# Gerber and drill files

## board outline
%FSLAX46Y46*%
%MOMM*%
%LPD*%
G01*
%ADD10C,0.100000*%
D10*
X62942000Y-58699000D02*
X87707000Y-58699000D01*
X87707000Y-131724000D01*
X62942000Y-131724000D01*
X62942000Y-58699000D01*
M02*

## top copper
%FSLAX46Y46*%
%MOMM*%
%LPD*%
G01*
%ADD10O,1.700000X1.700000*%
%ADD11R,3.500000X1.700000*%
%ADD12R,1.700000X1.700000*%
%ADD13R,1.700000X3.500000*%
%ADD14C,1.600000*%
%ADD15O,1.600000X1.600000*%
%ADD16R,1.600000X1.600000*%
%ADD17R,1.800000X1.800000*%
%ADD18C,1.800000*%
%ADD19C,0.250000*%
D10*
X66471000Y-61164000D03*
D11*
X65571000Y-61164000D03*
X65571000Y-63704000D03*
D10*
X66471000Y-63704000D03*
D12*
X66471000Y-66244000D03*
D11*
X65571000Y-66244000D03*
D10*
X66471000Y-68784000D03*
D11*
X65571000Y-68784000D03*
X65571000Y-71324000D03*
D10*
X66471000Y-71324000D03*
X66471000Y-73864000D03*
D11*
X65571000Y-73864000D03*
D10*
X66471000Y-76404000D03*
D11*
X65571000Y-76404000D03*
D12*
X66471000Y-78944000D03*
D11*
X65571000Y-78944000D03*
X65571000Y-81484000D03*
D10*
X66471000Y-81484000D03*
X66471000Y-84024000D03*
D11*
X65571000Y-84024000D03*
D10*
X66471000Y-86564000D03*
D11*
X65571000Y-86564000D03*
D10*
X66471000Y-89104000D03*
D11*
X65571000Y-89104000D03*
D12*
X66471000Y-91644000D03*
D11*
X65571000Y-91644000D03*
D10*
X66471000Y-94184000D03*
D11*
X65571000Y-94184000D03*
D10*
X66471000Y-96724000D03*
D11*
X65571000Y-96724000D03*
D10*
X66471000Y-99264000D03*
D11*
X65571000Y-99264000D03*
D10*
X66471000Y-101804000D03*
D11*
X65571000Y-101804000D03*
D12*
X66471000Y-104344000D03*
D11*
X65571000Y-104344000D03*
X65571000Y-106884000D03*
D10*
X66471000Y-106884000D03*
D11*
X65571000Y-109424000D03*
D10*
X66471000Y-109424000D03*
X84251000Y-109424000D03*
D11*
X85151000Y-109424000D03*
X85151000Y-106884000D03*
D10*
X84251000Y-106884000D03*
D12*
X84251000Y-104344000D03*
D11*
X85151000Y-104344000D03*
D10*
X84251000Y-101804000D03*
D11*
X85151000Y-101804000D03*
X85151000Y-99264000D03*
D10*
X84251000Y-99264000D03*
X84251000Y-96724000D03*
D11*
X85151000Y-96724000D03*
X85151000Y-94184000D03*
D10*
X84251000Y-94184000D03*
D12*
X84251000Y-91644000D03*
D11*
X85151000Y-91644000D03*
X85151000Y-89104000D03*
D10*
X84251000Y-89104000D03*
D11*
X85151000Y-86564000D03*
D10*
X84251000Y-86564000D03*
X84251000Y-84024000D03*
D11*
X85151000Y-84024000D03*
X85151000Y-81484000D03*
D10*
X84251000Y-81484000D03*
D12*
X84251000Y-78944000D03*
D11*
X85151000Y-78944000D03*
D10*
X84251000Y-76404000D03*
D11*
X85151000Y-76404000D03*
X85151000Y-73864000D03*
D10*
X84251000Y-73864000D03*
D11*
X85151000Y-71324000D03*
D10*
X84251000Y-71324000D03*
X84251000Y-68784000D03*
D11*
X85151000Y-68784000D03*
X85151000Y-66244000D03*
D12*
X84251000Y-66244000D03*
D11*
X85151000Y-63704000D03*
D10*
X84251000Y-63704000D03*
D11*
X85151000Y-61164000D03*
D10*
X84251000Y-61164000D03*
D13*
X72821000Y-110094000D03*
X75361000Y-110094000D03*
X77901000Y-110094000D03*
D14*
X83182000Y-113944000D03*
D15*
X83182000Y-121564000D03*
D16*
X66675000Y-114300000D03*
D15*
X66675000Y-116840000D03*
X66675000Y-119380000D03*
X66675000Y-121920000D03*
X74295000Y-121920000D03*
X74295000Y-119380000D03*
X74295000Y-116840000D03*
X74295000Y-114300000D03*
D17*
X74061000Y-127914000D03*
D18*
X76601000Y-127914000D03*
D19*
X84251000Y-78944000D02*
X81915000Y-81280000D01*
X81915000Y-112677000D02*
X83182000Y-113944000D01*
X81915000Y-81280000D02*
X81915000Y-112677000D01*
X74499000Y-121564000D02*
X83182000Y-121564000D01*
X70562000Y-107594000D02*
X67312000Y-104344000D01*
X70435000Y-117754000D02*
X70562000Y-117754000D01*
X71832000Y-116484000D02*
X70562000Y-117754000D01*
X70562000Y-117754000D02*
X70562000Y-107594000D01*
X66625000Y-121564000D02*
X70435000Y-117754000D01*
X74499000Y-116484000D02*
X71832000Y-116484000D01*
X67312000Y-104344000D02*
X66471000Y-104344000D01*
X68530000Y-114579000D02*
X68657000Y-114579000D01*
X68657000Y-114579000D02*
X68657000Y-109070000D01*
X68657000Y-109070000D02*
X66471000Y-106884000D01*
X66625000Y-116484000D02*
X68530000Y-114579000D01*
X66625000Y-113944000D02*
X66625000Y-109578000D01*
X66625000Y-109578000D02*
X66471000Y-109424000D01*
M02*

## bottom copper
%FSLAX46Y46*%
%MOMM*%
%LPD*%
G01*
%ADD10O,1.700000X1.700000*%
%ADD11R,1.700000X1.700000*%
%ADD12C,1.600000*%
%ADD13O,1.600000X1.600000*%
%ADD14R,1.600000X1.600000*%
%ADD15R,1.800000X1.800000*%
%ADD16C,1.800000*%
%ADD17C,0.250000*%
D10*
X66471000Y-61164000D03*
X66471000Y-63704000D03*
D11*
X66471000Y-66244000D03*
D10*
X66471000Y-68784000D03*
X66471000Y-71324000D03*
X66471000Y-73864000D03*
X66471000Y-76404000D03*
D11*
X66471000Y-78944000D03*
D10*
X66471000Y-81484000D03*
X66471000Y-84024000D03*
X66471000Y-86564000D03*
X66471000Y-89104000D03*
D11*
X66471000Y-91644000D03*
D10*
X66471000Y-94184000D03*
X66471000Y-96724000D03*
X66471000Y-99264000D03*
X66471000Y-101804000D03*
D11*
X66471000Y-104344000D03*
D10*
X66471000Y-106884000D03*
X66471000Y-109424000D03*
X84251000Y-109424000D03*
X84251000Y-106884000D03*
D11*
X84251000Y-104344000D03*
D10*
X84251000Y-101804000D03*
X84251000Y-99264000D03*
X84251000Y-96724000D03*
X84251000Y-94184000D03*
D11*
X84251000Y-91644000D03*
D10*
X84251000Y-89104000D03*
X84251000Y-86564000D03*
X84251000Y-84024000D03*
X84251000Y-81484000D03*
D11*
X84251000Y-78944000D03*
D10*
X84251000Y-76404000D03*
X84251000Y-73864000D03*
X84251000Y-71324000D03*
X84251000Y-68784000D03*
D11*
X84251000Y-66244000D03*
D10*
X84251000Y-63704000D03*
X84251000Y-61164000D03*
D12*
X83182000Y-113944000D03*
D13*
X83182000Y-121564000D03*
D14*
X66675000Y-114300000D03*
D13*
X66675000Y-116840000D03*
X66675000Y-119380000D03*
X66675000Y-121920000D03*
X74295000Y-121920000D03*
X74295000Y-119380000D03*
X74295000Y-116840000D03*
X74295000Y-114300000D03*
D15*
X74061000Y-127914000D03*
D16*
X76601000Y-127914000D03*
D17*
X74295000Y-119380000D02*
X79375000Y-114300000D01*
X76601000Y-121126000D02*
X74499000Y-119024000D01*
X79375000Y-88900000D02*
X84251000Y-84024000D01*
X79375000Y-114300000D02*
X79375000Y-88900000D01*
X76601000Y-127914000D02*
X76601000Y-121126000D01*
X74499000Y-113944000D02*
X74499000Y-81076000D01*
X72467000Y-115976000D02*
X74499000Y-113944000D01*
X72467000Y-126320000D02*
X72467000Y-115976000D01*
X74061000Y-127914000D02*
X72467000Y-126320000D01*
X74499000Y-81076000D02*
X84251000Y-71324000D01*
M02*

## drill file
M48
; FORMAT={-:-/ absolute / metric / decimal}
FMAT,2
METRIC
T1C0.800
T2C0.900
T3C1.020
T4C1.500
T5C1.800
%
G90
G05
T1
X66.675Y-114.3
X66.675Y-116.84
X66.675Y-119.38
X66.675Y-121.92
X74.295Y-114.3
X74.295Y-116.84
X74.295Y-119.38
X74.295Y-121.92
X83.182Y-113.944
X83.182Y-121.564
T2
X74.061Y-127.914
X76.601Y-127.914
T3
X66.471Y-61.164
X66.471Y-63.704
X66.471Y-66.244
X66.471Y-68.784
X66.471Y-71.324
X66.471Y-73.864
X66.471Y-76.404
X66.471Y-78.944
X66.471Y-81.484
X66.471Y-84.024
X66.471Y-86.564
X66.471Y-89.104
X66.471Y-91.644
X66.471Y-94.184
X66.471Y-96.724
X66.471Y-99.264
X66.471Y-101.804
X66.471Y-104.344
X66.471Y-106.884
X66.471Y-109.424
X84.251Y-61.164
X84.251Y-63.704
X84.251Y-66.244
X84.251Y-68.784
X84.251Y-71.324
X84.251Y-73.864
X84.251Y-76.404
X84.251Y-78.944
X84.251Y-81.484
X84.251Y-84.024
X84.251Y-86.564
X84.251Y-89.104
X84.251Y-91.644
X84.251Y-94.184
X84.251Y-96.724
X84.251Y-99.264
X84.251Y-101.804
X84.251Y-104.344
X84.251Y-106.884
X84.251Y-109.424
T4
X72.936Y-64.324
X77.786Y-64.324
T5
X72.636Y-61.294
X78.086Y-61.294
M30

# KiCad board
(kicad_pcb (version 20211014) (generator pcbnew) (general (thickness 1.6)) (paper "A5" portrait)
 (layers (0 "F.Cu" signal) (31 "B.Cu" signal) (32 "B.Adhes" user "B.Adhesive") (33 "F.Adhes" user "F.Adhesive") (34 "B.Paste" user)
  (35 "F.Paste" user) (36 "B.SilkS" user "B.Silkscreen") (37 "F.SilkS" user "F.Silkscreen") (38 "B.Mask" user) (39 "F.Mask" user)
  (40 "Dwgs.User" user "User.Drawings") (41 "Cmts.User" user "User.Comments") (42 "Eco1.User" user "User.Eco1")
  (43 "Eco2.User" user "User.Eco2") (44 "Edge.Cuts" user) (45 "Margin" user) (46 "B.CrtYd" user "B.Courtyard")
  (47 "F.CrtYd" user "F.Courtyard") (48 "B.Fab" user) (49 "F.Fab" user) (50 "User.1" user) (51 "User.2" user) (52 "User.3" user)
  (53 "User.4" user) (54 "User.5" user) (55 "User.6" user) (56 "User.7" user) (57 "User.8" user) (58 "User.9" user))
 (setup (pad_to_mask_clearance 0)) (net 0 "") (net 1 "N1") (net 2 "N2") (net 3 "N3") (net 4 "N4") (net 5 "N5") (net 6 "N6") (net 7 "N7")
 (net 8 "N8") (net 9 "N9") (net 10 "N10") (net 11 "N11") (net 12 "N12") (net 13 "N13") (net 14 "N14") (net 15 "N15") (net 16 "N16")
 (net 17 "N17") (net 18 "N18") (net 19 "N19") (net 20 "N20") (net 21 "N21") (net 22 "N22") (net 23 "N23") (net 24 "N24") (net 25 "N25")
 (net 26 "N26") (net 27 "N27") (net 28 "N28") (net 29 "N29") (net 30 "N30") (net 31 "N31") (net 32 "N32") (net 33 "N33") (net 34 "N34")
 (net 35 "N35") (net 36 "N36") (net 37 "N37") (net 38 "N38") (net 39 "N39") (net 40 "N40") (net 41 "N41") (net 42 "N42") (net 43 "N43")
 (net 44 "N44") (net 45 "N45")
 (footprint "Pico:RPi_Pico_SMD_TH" (layer "F.Cu") (at 75.361 85.294)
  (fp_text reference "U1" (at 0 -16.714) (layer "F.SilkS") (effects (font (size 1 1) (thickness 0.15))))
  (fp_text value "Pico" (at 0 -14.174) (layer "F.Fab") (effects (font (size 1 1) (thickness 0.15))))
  (pad "" np_thru_hole oval (at -2.425 -20.97) (size 1.5 1.5) (drill 1.5) (layers *.Cu *.Mask))
  (pad "" np_thru_hole oval (at 2.725 -24) (size 1.8 1.8) (drill 1.8) (layers *.Cu *.Mask))
  (pad "" np_thru_hole oval (at 2.425 -20.97) (size 1.5 1.5) (drill 1.5) (layers *.Cu *.Mask))
  (pad "" np_thru_hole oval (at -2.725 -24) (size 1.8 1.8) (drill 1.8) (layers *.Cu *.Mask))
  (pad "1" thru_hole oval (at -8.89 -24.13) (size 1.7 1.7) (drill 1.02) (layers *.Cu *.Mask) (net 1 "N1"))
  (pad "1" smd rect (at -8.89 -24.13) (size 3.5 1.7) (drill (offset -0.9 0)) (layers "F.Cu" "F.Mask") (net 1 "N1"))
  (pad "2" smd rect (at -8.89 -21.59) (size 3.5 1.7) (drill (offset -0.9 0)) (layers "F.Cu" "F.Mask") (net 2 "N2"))
  (pad "2" thru_hole oval (at -8.89 -21.59) (size 1.7 1.7) (drill 1.02) (layers *.Cu *.Mask) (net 2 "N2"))
  (pad "3" thru_hole rect (at -8.89 -19.05) (size 1.7 1.7) (drill 1.02) (layers *.Cu *.Mask) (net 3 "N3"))
  (pad "3" smd rect (at -8.89 -19.05) (size 3.5 1.7) (drill (offset -0.9 0)) (layers "F.Cu" "F.Mask") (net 3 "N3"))
  (pad "4" thru_hole oval (at -8.89 -16.51) (size 1.7 1.7) (drill 1.02) (layers *.Cu *.Mask) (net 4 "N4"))
  (pad "4" smd rect (at -8.89 -16.51) (size 3.5 1.7) (drill (offset -0.9 0)) (layers "F.Cu" "F.Mask") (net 4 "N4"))
  (pad "5" smd rect (at -8.89 -13.97) (size 3.5 1.7) (drill (offset -0.9 0)) (layers "F.Cu" "F.Mask") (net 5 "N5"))
  (pad "5" thru_hole oval (at -8.89 -13.97) (size 1.7 1.7) (drill 1.02) (layers *.Cu *.Mask) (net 5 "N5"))
  (pad "6" thru_hole oval (at -8.89 -11.43) (size 1.7 1.7) (drill 1.02) (layers *.Cu *.Mask) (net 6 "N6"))
  (pad "6" smd rect (at -8.89 -11.43) (size 3.5 1.7) (drill (offset -0.9 0)) (layers "F.Cu" "F.Mask") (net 6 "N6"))
  (pad "7" thru_hole oval (at -8.89 -8.89) (size 1.7 1.7) (drill 1.02) (layers *.Cu *.Mask) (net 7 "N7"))
  (pad "7" smd rect (at -8.89 -8.89) (size 3.5 1.7) (drill (offset -0.9 0)) (layers "F.Cu" "F.Mask") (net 7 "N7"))
  (pad "8" thru_hole rect (at -8.89 -6.35) (size 1.7 1.7) (drill 1.02) (layers *.Cu *.Mask) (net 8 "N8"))
  (pad "8" smd rect (at -8.89 -6.35) (size 3.5 1.7) (drill (offset -0.9 0)) (layers "F.Cu" "F.Mask") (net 8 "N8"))
  (pad "9" smd rect (at -8.89 -3.81) (size 3.5 1.7) (drill (offset -0.9 0)) (layers "F.Cu" "F.Mask") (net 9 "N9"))
  (pad "9" thru_hole oval (at -8.89 -3.81) (size 1.7 1.7) (drill 1.02) (layers *.Cu *.Mask) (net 9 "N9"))
  (pad "10" thru_hole oval (at -8.89 -1.27) (size 1.7 1.7) (drill 1.02) (layers *.Cu *.Mask) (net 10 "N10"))
  (pad "10" smd rect (at -8.89 -1.27) (size 3.5 1.7) (drill (offset -0.9 0)) (layers "F.Cu" "F.Mask") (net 10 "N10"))
  (pad "11" thru_hole oval (at -8.89 1.27) (size 1.7 1.7) (drill 1.02) (layers *.Cu *.Mask) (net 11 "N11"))
  (pad "11" smd rect (at -8.89 1.27) (size 3.5 1.7) (drill (offset -0.9 0)) (layers "F.Cu" "F.Mask") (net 11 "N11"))
  (pad "12" thru_hole oval (at -8.89 3.81) (size 1.7 1.7) (drill 1.02) (layers *.Cu *.Mask) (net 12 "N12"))
  (pad "12" smd rect (at -8.89 3.81) (size 3.5 1.7) (drill (offset -0.9 0)) (layers "F.Cu" "F.Mask") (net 12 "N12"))
  (pad "13" thru_hole rect (at -8.89 6.35) (size 1.7 1.7) (drill 1.02) (layers *.Cu *.Mask) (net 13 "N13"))
  (pad "13" smd rect (at -8.89 6.35) (size 3.5 1.7) (drill (offset -0.9 0)) (layers "F.Cu" "F.Mask") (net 13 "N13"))
  (pad "14" thru_hole oval (at -8.89 8.89) (size 1.7 1.7) (drill 1.02) (layers *.Cu *.Mask) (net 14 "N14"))
  (pad "14" smd rect (at -8.89 8.89) (size 3.5 1.7) (drill (offset -0.9 0)) (layers "F.Cu" "F.Mask") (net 14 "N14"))
  (pad "15" thru_hole oval (at -8.89 11.43) (size 1.7 1.7) (drill 1.02) (layers *.Cu *.Mask) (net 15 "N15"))
  (pad "15" smd rect (at -8.89 11.43) (size 3.5 1.7) (drill (offset -0.9 0)) (layers "F.Cu" "F.Mask") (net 15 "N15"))
  (pad "16" thru_hole oval (at -8.89 13.97) (size 1.7 1.7) (drill 1.02) (layers *.Cu *.Mask) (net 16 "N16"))
  (pad "16" smd rect (at -8.89 13.97) (size 3.5 1.7) (drill (offset -0.9 0)) (layers "F.Cu" "F.Mask") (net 16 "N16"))
  (pad "17" thru_hole oval (at -8.89 16.51) (size 1.7 1.7) (drill 1.02) (layers *.Cu *.Mask) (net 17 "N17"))
  (pad "17" smd rect (at -8.89 16.51) (size 3.5 1.7) (drill (offset -0.9 0)) (layers "F.Cu" "F.Mask") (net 17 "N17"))
  (pad "18" thru_hole rect (at -8.89 19.05) (size 1.7 1.7) (drill 1.02) (layers *.Cu *.Mask) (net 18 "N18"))
  (pad "18" smd rect (at -8.89 19.05) (size 3.5 1.7) (drill (offset -0.9 0)) (layers "F.Cu" "F.Mask") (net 18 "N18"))
  (pad "19" smd rect (at -8.89 21.59) (size 3.5 1.7) (drill (offset -0.9 0)) (layers "F.Cu" "F.Mask") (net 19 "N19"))
  (pad "19" thru_hole oval (at -8.89 21.59) (size 1.7 1.7) (drill 1.02) (layers *.Cu *.Mask) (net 19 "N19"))
  (pad "20" smd rect (at -8.89 24.13) (size 3.5 1.7) (drill (offset -0.9 0)) (layers "F.Cu" "F.Mask") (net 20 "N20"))
  (pad "20" thru_hole oval (at -8.89 24.13) (size 1.7 1.7) (drill 1.02) (layers *.Cu *.Mask) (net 20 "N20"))
  (pad "21" thru_hole oval (at 8.89 24.13) (size 1.7 1.7) (drill 1.02) (layers *.Cu *.Mask) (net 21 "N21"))
  (pad "21" smd rect (at 8.89 24.13) (size 3.5 1.7) (drill (offset 0.9 0)) (layers "F.Cu" "F.Mask") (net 21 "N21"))
  (pad "22" smd rect (at 8.89 21.59) (size 3.5 1.7) (drill (offset 0.9 0)) (layers "F.Cu" "F.Mask") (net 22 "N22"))
  (pad "22" thru_hole oval (at 8.89 21.59) (size 1.7 1.7) (drill 1.02) (layers *.Cu *.Mask) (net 22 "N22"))
  (pad "23" thru_hole rect (at 8.89 19.05) (size 1.7 1.7) (drill 1.02) (layers *.Cu *.Mask) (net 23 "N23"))
  (pad "23" smd rect (at 8.89 19.05) (size 3.5 1.7) (drill (offset 0.9 0)) (layers "F.Cu" "F.Mask") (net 23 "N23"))
  (pad "24" thru_hole oval (at 8.89 16.51) (size 1.7 1.7) (drill 1.02) (layers *.Cu *.Mask) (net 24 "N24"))
  (pad "24" smd rect (at 8.89 16.51) (size 3.5 1.7) (drill (offset 0.9 0)) (layers "F.Cu" "F.Mask") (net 24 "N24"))
  (pad "25" smd rect (at 8.89 13.97) (size 3.5 1.7) (drill (offset 0.9 0)) (layers "F.Cu" "F.Mask") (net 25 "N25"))
  (pad "25" thru_hole oval (at 8.89 13.97) (size 1.7 1.7) (drill 1.02) (layers *.Cu *.Mask) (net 25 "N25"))
  (pad "26" thru_hole oval (at 8.89 11.43) (size 1.7 1.7) (drill 1.02) (layers *.Cu *.Mask) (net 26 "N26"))
  (pad "26" smd rect (at 8.89 11.43) (size 3.5 1.7) (drill (offset 0.9 0)) (layers "F.Cu" "F.Mask") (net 26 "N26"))
  (pad "27" smd rect (at 8.89 8.89) (size 3.5 1.7) (drill (offset 0.9 0)) (layers "F.Cu" "F.Mask") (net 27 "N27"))
  (pad "27" thru_hole oval (at 8.89 8.89) (size 1.7 1.7) (drill 1.02) (layers *.Cu *.Mask) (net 27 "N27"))
  (pad "28" thru_hole rect (at 8.89 6.35) (size 1.7 1.7) (drill 1.02) (layers *.Cu *.Mask) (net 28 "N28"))
  (pad "28" smd rect (at 8.89 6.35) (size 3.5 1.7) (drill (offset 0.9 0)) (layers "F.Cu" "F.Mask") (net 28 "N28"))
  (pad "29" smd rect (at 8.89 3.81) (size 3.5 1.7) (drill (offset 0.9 0)) (layers "F.Cu" "F.Mask") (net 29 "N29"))
  (pad "29" thru_hole oval (at 8.89 3.81) (size 1.7 1.7) (drill 1.02) (layers *.Cu *.Mask) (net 29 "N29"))
  (pad "30" smd rect (at 8.89 1.27) (size 3.5 1.7) (drill (offset 0.9 0)) (layers "F.Cu" "F.Mask") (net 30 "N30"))
  (pad "30" thru_hole oval (at 8.89 1.27) (size 1.7 1.7) (drill 1.02) (layers *.Cu *.Mask) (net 30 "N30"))
  (pad "31" thru_hole oval (at 8.89 -1.27) (size 1.7 1.7) (drill 1.02) (layers *.Cu *.Mask) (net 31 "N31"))
  (pad "31" smd rect (at 8.89 -1.27) (size 3.5 1.7) (drill (offset 0.9 0)) (layers "F.Cu" "F.Mask") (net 31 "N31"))
  (pad "32" smd rect (at 8.89 -3.81) (size 3.5 1.7) (drill (offset 0.9 0)) (layers "F.Cu" "F.Mask") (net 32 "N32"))
  (pad "32" thru_hole oval (at 8.89 -3.81) (size 1.7 1.7) (drill 1.02) (layers *.Cu *.Mask) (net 32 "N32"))
  (pad "33" thru_hole rect (at 8.89 -6.35) (size 1.7 1.7) (drill 1.02) (layers *.Cu *.Mask) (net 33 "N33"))
  (pad "33" smd rect (at 8.89 -6.35) (size 3.5 1.7) (drill (offset 0.9 0)) (layers "F.Cu" "F.Mask") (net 33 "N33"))
  (pad "34" thru_hole oval (at 8.89 -8.89) (size 1.7 1.7) (drill 1.02) (layers *.Cu *.Mask) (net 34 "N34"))
  (pad "34" smd rect (at 8.89 -8.89) (size 3.5 1.7) (drill (offset 0.9 0)) (layers "F.Cu" "F.Mask") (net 34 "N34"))
  (pad "35" smd rect (at 8.89 -11.43) (size 3.5 1.7) (drill (offset 0.9 0)) (layers "F.Cu" "F.Mask") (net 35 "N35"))
  (pad "35" thru_hole oval (at 8.89 -11.43) (size 1.7 1.7) (drill 1.02) (layers *.Cu *.Mask) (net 35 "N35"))
  (pad "36" smd rect (at 8.89 -13.97) (size 3.5 1.7) (drill (offset 0.9 0)) (layers "F.Cu" "F.Mask") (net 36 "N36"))
  (pad "36" thru_hole oval (at 8.89 -13.97) (size 1.7 1.7) (drill 1.02) (layers *.Cu *.Mask) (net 36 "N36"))
  (pad "37" thru_hole oval (at 8.89 -16.51) (size 1.7 1.7) (drill 1.02) (layers *.Cu *.Mask) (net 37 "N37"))
  (pad "37" smd rect (at 8.89 -16.51) (size 3.5 1.7) (drill (offset 0.9 0)) (layers "F.Cu" "F.Mask") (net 37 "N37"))
  (pad "38" smd rect (at 8.89 -19.05) (size 3.5 1.7) (drill (offset 0.9 0)) (layers "F.Cu" "F.Mask") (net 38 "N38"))
  (pad "38" thru_hole rect (at 8.89 -19.05) (size 1.7 1.7) (drill 1.02) (layers *.Cu *.Mask) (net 38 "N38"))
  (pad "39" smd rect (at 8.89 -21.59) (size 3.5 1.7) (drill (offset 0.9 0)) (layers "F.Cu" "F.Mask") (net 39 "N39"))
  (pad "39" thru_hole oval (at 8.89 -21.59) (size 1.7 1.7) (drill 1.02) (layers *.Cu *.Mask) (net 39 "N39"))
  (pad "40" smd rect (at 8.89 -24.13) (size 3.5 1.7) (drill (offset 0.9 0)) (layers "F.Cu" "F.Mask") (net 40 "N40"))
  (pad "40" thru_hole oval (at 8.89 -24.13) (size 1.7 1.7) (drill 1.02) (layers *.Cu *.Mask) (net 40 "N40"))
  (pad "41" smd rect (at -2.54 23.9 90) (size 3.5 1.7) (drill (offset -0.9 0)) (layers "F.Cu" "F.Mask") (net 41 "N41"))
  (pad "42" smd rect (at 0 23.9 90) (size 3.5 1.7) (drill (offset -0.9 0)) (layers "F.Cu" "F.Mask") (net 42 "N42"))
  (pad "43" smd rect (at 2.54 23.9 90) (size 3.5 1.7) (drill (offset -0.9 0)) (layers "F.Cu" "F.Mask") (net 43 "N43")))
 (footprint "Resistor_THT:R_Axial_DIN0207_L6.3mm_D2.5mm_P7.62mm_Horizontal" (layer "F.Cu") (at 83.182 113.944 -90)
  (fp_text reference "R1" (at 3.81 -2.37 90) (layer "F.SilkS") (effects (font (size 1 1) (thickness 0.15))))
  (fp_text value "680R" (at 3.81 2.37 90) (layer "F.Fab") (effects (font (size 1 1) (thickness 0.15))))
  (pad "1" thru_hole circle (at 0 0 270) (size 1.6 1.6) (drill 0.8) (layers *.Cu *.Mask) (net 33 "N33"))
  (pad "2" thru_hole oval (at 7.62 0 270) (size 1.6 1.6) (drill 0.8) (layers *.Cu *.Mask) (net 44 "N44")))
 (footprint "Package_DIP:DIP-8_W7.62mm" (layer "F.Cu") (at 66.675 114.3)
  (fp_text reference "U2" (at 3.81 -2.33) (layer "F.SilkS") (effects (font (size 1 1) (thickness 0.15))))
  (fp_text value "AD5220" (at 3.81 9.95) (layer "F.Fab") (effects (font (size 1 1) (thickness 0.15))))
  (pad "1" thru_hole rect (at 0 0) (size 1.6 1.6) (drill 0.8) (layers *.Cu *.Mask) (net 20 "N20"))
  (pad "2" thru_hole oval (at 0 2.54) (size 1.6 1.6) (drill 0.8) (layers *.Cu *.Mask) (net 19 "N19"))
  (pad "3" thru_hole oval (at 0 5.08) (size 1.6 1.6) (drill 0.8) (layers *.Cu *.Mask) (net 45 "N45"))
  (pad "4" thru_hole oval (at 0 7.62) (size 1.6 1.6) (drill 0.8) (layers *.Cu *.Mask) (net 18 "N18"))
  (pad "5" thru_hole oval (at 7.62 7.62) (size 1.6 1.6) (drill 0.8) (layers *.Cu *.Mask) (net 44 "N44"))
  (pad "6" thru_hole oval (at 7.62 5.08) (size 1.6 1.6) (drill 0.8) (layers *.Cu *.Mask) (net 31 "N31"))
  (pad "7" thru_hole oval (at 7.62 2.54) (size 1.6 1.6) (drill 0.8) (layers *.Cu *.Mask) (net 18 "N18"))
  (pad "8" thru_hole oval (at 7.62 0) (size 1.6 1.6) (drill 0.8) (layers *.Cu *.Mask) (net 36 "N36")))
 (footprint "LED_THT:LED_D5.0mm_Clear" (layer "F.Cu") (at 74.061 127.914)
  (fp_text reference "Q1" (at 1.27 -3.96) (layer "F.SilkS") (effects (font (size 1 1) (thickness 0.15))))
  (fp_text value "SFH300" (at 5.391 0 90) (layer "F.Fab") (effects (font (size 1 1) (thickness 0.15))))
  (pad "1" thru_hole rect (at 0 0) (size 1.8 1.8) (drill 0.9) (layers *.Cu *.Mask) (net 36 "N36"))
  (pad "2" thru_hole circle (at 2.54 0) (size 1.8 1.8) (drill 0.9) (layers *.Cu *.Mask) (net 31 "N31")))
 (gr_rect (start 62.942 58.699) (end 87.707 131.724) (layer "Edge.Cuts") (width 0.1) (fill none))
 (segment (start 84.251 78.944) (end 81.915 81.28) (width 0.25) (layer "F.Cu") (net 33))
 (segment (start 81.915 112.677) (end 83.182 113.944) (width 0.25) (layer "F.Cu") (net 33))
 (segment (start 81.915 81.28) (end 81.915 112.677) (width 0.25) (layer "F.Cu") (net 33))
 (segment (start 74.499 121.564) (end 83.182 121.564) (width 0.25) (layer "F.Cu") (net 44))
 (segment (start 70.562 107.594) (end 67.312 104.344) (width 0.25) (layer "F.Cu") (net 18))
 (segment (start 70.435 117.754) (end 70.562 117.754) (width 0.25) (layer "F.Cu") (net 18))
 (segment (start 71.832 116.484) (end 70.562 117.754) (width 0.25) (layer "F.Cu") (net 18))
 (segment (start 70.562 117.754) (end 70.562 107.594) (width 0.25) (layer "F.Cu") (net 18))
 (segment (start 66.625 121.564) (end 70.435 117.754) (width 0.25) (layer "F.Cu") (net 18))
 (segment (start 74.499 116.484) (end 71.832 116.484) (width 0.25) (layer "F.Cu") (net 18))
 (segment (start 67.312 104.344) (end 66.471 104.344) (width 0.25) (layer "F.Cu") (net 18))
 (segment (start 68.53 114.579) (end 68.657 114.579) (width 0.25) (layer "F.Cu") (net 19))
 (segment (start 68.657 114.579) (end 68.657 109.07) (width 0.25) (layer "F.Cu") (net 19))
 (segment (start 68.657 109.07) (end 66.471 106.884) (width 0.25) (layer "F.Cu") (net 19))
 (segment (start 66.625 116.484) (end 68.53 114.579) (width 0.25) (layer "F.Cu") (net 19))
 (segment (start 74.295 119.38) (end 79.375 114.3) (width 0.25) (layer "B.Cu") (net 31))
 (segment (start 76.601 121.126) (end 74.499 119.024) (width 0.25) (layer "B.Cu") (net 31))
 (segment (start 79.375 88.9) (end 84.251 84.024) (width 0.25) (layer "B.Cu") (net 31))
 (segment (start 79.375 114.3) (end 79.375 88.9) (width 0.25) (layer "B.Cu") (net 31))
 (segment (start 76.601 127.914) (end 76.601 121.126) (width 0.25) (layer "B.Cu") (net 31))
 (segment (start 74.499 113.944) (end 74.499 81.076) (width 0.25) (layer "B.Cu") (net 36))
 (segment (start 72.467 115.976) (end 74.499 113.944) (width 0.25) (layer "B.Cu") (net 36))
 (segment (start 72.467 126.32) (end 72.467 115.976) (width 0.25) (layer "B.Cu") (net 36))
 (segment (start 74.061 127.914) (end 72.467 126.32) (width 0.25) (layer "B.Cu") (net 36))
 (segment (start 74.499 81.076) (end 84.251 71.324) (width 0.25) (layer "B.Cu") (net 36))
 (segment (start 66.625 113.944) (end 66.625 109.578) (width 0.25) (layer "F.Cu") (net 20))
 (segment (start 66.625 109.578) (end 66.471 109.424) (width 0.25) (layer "F.Cu") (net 20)))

